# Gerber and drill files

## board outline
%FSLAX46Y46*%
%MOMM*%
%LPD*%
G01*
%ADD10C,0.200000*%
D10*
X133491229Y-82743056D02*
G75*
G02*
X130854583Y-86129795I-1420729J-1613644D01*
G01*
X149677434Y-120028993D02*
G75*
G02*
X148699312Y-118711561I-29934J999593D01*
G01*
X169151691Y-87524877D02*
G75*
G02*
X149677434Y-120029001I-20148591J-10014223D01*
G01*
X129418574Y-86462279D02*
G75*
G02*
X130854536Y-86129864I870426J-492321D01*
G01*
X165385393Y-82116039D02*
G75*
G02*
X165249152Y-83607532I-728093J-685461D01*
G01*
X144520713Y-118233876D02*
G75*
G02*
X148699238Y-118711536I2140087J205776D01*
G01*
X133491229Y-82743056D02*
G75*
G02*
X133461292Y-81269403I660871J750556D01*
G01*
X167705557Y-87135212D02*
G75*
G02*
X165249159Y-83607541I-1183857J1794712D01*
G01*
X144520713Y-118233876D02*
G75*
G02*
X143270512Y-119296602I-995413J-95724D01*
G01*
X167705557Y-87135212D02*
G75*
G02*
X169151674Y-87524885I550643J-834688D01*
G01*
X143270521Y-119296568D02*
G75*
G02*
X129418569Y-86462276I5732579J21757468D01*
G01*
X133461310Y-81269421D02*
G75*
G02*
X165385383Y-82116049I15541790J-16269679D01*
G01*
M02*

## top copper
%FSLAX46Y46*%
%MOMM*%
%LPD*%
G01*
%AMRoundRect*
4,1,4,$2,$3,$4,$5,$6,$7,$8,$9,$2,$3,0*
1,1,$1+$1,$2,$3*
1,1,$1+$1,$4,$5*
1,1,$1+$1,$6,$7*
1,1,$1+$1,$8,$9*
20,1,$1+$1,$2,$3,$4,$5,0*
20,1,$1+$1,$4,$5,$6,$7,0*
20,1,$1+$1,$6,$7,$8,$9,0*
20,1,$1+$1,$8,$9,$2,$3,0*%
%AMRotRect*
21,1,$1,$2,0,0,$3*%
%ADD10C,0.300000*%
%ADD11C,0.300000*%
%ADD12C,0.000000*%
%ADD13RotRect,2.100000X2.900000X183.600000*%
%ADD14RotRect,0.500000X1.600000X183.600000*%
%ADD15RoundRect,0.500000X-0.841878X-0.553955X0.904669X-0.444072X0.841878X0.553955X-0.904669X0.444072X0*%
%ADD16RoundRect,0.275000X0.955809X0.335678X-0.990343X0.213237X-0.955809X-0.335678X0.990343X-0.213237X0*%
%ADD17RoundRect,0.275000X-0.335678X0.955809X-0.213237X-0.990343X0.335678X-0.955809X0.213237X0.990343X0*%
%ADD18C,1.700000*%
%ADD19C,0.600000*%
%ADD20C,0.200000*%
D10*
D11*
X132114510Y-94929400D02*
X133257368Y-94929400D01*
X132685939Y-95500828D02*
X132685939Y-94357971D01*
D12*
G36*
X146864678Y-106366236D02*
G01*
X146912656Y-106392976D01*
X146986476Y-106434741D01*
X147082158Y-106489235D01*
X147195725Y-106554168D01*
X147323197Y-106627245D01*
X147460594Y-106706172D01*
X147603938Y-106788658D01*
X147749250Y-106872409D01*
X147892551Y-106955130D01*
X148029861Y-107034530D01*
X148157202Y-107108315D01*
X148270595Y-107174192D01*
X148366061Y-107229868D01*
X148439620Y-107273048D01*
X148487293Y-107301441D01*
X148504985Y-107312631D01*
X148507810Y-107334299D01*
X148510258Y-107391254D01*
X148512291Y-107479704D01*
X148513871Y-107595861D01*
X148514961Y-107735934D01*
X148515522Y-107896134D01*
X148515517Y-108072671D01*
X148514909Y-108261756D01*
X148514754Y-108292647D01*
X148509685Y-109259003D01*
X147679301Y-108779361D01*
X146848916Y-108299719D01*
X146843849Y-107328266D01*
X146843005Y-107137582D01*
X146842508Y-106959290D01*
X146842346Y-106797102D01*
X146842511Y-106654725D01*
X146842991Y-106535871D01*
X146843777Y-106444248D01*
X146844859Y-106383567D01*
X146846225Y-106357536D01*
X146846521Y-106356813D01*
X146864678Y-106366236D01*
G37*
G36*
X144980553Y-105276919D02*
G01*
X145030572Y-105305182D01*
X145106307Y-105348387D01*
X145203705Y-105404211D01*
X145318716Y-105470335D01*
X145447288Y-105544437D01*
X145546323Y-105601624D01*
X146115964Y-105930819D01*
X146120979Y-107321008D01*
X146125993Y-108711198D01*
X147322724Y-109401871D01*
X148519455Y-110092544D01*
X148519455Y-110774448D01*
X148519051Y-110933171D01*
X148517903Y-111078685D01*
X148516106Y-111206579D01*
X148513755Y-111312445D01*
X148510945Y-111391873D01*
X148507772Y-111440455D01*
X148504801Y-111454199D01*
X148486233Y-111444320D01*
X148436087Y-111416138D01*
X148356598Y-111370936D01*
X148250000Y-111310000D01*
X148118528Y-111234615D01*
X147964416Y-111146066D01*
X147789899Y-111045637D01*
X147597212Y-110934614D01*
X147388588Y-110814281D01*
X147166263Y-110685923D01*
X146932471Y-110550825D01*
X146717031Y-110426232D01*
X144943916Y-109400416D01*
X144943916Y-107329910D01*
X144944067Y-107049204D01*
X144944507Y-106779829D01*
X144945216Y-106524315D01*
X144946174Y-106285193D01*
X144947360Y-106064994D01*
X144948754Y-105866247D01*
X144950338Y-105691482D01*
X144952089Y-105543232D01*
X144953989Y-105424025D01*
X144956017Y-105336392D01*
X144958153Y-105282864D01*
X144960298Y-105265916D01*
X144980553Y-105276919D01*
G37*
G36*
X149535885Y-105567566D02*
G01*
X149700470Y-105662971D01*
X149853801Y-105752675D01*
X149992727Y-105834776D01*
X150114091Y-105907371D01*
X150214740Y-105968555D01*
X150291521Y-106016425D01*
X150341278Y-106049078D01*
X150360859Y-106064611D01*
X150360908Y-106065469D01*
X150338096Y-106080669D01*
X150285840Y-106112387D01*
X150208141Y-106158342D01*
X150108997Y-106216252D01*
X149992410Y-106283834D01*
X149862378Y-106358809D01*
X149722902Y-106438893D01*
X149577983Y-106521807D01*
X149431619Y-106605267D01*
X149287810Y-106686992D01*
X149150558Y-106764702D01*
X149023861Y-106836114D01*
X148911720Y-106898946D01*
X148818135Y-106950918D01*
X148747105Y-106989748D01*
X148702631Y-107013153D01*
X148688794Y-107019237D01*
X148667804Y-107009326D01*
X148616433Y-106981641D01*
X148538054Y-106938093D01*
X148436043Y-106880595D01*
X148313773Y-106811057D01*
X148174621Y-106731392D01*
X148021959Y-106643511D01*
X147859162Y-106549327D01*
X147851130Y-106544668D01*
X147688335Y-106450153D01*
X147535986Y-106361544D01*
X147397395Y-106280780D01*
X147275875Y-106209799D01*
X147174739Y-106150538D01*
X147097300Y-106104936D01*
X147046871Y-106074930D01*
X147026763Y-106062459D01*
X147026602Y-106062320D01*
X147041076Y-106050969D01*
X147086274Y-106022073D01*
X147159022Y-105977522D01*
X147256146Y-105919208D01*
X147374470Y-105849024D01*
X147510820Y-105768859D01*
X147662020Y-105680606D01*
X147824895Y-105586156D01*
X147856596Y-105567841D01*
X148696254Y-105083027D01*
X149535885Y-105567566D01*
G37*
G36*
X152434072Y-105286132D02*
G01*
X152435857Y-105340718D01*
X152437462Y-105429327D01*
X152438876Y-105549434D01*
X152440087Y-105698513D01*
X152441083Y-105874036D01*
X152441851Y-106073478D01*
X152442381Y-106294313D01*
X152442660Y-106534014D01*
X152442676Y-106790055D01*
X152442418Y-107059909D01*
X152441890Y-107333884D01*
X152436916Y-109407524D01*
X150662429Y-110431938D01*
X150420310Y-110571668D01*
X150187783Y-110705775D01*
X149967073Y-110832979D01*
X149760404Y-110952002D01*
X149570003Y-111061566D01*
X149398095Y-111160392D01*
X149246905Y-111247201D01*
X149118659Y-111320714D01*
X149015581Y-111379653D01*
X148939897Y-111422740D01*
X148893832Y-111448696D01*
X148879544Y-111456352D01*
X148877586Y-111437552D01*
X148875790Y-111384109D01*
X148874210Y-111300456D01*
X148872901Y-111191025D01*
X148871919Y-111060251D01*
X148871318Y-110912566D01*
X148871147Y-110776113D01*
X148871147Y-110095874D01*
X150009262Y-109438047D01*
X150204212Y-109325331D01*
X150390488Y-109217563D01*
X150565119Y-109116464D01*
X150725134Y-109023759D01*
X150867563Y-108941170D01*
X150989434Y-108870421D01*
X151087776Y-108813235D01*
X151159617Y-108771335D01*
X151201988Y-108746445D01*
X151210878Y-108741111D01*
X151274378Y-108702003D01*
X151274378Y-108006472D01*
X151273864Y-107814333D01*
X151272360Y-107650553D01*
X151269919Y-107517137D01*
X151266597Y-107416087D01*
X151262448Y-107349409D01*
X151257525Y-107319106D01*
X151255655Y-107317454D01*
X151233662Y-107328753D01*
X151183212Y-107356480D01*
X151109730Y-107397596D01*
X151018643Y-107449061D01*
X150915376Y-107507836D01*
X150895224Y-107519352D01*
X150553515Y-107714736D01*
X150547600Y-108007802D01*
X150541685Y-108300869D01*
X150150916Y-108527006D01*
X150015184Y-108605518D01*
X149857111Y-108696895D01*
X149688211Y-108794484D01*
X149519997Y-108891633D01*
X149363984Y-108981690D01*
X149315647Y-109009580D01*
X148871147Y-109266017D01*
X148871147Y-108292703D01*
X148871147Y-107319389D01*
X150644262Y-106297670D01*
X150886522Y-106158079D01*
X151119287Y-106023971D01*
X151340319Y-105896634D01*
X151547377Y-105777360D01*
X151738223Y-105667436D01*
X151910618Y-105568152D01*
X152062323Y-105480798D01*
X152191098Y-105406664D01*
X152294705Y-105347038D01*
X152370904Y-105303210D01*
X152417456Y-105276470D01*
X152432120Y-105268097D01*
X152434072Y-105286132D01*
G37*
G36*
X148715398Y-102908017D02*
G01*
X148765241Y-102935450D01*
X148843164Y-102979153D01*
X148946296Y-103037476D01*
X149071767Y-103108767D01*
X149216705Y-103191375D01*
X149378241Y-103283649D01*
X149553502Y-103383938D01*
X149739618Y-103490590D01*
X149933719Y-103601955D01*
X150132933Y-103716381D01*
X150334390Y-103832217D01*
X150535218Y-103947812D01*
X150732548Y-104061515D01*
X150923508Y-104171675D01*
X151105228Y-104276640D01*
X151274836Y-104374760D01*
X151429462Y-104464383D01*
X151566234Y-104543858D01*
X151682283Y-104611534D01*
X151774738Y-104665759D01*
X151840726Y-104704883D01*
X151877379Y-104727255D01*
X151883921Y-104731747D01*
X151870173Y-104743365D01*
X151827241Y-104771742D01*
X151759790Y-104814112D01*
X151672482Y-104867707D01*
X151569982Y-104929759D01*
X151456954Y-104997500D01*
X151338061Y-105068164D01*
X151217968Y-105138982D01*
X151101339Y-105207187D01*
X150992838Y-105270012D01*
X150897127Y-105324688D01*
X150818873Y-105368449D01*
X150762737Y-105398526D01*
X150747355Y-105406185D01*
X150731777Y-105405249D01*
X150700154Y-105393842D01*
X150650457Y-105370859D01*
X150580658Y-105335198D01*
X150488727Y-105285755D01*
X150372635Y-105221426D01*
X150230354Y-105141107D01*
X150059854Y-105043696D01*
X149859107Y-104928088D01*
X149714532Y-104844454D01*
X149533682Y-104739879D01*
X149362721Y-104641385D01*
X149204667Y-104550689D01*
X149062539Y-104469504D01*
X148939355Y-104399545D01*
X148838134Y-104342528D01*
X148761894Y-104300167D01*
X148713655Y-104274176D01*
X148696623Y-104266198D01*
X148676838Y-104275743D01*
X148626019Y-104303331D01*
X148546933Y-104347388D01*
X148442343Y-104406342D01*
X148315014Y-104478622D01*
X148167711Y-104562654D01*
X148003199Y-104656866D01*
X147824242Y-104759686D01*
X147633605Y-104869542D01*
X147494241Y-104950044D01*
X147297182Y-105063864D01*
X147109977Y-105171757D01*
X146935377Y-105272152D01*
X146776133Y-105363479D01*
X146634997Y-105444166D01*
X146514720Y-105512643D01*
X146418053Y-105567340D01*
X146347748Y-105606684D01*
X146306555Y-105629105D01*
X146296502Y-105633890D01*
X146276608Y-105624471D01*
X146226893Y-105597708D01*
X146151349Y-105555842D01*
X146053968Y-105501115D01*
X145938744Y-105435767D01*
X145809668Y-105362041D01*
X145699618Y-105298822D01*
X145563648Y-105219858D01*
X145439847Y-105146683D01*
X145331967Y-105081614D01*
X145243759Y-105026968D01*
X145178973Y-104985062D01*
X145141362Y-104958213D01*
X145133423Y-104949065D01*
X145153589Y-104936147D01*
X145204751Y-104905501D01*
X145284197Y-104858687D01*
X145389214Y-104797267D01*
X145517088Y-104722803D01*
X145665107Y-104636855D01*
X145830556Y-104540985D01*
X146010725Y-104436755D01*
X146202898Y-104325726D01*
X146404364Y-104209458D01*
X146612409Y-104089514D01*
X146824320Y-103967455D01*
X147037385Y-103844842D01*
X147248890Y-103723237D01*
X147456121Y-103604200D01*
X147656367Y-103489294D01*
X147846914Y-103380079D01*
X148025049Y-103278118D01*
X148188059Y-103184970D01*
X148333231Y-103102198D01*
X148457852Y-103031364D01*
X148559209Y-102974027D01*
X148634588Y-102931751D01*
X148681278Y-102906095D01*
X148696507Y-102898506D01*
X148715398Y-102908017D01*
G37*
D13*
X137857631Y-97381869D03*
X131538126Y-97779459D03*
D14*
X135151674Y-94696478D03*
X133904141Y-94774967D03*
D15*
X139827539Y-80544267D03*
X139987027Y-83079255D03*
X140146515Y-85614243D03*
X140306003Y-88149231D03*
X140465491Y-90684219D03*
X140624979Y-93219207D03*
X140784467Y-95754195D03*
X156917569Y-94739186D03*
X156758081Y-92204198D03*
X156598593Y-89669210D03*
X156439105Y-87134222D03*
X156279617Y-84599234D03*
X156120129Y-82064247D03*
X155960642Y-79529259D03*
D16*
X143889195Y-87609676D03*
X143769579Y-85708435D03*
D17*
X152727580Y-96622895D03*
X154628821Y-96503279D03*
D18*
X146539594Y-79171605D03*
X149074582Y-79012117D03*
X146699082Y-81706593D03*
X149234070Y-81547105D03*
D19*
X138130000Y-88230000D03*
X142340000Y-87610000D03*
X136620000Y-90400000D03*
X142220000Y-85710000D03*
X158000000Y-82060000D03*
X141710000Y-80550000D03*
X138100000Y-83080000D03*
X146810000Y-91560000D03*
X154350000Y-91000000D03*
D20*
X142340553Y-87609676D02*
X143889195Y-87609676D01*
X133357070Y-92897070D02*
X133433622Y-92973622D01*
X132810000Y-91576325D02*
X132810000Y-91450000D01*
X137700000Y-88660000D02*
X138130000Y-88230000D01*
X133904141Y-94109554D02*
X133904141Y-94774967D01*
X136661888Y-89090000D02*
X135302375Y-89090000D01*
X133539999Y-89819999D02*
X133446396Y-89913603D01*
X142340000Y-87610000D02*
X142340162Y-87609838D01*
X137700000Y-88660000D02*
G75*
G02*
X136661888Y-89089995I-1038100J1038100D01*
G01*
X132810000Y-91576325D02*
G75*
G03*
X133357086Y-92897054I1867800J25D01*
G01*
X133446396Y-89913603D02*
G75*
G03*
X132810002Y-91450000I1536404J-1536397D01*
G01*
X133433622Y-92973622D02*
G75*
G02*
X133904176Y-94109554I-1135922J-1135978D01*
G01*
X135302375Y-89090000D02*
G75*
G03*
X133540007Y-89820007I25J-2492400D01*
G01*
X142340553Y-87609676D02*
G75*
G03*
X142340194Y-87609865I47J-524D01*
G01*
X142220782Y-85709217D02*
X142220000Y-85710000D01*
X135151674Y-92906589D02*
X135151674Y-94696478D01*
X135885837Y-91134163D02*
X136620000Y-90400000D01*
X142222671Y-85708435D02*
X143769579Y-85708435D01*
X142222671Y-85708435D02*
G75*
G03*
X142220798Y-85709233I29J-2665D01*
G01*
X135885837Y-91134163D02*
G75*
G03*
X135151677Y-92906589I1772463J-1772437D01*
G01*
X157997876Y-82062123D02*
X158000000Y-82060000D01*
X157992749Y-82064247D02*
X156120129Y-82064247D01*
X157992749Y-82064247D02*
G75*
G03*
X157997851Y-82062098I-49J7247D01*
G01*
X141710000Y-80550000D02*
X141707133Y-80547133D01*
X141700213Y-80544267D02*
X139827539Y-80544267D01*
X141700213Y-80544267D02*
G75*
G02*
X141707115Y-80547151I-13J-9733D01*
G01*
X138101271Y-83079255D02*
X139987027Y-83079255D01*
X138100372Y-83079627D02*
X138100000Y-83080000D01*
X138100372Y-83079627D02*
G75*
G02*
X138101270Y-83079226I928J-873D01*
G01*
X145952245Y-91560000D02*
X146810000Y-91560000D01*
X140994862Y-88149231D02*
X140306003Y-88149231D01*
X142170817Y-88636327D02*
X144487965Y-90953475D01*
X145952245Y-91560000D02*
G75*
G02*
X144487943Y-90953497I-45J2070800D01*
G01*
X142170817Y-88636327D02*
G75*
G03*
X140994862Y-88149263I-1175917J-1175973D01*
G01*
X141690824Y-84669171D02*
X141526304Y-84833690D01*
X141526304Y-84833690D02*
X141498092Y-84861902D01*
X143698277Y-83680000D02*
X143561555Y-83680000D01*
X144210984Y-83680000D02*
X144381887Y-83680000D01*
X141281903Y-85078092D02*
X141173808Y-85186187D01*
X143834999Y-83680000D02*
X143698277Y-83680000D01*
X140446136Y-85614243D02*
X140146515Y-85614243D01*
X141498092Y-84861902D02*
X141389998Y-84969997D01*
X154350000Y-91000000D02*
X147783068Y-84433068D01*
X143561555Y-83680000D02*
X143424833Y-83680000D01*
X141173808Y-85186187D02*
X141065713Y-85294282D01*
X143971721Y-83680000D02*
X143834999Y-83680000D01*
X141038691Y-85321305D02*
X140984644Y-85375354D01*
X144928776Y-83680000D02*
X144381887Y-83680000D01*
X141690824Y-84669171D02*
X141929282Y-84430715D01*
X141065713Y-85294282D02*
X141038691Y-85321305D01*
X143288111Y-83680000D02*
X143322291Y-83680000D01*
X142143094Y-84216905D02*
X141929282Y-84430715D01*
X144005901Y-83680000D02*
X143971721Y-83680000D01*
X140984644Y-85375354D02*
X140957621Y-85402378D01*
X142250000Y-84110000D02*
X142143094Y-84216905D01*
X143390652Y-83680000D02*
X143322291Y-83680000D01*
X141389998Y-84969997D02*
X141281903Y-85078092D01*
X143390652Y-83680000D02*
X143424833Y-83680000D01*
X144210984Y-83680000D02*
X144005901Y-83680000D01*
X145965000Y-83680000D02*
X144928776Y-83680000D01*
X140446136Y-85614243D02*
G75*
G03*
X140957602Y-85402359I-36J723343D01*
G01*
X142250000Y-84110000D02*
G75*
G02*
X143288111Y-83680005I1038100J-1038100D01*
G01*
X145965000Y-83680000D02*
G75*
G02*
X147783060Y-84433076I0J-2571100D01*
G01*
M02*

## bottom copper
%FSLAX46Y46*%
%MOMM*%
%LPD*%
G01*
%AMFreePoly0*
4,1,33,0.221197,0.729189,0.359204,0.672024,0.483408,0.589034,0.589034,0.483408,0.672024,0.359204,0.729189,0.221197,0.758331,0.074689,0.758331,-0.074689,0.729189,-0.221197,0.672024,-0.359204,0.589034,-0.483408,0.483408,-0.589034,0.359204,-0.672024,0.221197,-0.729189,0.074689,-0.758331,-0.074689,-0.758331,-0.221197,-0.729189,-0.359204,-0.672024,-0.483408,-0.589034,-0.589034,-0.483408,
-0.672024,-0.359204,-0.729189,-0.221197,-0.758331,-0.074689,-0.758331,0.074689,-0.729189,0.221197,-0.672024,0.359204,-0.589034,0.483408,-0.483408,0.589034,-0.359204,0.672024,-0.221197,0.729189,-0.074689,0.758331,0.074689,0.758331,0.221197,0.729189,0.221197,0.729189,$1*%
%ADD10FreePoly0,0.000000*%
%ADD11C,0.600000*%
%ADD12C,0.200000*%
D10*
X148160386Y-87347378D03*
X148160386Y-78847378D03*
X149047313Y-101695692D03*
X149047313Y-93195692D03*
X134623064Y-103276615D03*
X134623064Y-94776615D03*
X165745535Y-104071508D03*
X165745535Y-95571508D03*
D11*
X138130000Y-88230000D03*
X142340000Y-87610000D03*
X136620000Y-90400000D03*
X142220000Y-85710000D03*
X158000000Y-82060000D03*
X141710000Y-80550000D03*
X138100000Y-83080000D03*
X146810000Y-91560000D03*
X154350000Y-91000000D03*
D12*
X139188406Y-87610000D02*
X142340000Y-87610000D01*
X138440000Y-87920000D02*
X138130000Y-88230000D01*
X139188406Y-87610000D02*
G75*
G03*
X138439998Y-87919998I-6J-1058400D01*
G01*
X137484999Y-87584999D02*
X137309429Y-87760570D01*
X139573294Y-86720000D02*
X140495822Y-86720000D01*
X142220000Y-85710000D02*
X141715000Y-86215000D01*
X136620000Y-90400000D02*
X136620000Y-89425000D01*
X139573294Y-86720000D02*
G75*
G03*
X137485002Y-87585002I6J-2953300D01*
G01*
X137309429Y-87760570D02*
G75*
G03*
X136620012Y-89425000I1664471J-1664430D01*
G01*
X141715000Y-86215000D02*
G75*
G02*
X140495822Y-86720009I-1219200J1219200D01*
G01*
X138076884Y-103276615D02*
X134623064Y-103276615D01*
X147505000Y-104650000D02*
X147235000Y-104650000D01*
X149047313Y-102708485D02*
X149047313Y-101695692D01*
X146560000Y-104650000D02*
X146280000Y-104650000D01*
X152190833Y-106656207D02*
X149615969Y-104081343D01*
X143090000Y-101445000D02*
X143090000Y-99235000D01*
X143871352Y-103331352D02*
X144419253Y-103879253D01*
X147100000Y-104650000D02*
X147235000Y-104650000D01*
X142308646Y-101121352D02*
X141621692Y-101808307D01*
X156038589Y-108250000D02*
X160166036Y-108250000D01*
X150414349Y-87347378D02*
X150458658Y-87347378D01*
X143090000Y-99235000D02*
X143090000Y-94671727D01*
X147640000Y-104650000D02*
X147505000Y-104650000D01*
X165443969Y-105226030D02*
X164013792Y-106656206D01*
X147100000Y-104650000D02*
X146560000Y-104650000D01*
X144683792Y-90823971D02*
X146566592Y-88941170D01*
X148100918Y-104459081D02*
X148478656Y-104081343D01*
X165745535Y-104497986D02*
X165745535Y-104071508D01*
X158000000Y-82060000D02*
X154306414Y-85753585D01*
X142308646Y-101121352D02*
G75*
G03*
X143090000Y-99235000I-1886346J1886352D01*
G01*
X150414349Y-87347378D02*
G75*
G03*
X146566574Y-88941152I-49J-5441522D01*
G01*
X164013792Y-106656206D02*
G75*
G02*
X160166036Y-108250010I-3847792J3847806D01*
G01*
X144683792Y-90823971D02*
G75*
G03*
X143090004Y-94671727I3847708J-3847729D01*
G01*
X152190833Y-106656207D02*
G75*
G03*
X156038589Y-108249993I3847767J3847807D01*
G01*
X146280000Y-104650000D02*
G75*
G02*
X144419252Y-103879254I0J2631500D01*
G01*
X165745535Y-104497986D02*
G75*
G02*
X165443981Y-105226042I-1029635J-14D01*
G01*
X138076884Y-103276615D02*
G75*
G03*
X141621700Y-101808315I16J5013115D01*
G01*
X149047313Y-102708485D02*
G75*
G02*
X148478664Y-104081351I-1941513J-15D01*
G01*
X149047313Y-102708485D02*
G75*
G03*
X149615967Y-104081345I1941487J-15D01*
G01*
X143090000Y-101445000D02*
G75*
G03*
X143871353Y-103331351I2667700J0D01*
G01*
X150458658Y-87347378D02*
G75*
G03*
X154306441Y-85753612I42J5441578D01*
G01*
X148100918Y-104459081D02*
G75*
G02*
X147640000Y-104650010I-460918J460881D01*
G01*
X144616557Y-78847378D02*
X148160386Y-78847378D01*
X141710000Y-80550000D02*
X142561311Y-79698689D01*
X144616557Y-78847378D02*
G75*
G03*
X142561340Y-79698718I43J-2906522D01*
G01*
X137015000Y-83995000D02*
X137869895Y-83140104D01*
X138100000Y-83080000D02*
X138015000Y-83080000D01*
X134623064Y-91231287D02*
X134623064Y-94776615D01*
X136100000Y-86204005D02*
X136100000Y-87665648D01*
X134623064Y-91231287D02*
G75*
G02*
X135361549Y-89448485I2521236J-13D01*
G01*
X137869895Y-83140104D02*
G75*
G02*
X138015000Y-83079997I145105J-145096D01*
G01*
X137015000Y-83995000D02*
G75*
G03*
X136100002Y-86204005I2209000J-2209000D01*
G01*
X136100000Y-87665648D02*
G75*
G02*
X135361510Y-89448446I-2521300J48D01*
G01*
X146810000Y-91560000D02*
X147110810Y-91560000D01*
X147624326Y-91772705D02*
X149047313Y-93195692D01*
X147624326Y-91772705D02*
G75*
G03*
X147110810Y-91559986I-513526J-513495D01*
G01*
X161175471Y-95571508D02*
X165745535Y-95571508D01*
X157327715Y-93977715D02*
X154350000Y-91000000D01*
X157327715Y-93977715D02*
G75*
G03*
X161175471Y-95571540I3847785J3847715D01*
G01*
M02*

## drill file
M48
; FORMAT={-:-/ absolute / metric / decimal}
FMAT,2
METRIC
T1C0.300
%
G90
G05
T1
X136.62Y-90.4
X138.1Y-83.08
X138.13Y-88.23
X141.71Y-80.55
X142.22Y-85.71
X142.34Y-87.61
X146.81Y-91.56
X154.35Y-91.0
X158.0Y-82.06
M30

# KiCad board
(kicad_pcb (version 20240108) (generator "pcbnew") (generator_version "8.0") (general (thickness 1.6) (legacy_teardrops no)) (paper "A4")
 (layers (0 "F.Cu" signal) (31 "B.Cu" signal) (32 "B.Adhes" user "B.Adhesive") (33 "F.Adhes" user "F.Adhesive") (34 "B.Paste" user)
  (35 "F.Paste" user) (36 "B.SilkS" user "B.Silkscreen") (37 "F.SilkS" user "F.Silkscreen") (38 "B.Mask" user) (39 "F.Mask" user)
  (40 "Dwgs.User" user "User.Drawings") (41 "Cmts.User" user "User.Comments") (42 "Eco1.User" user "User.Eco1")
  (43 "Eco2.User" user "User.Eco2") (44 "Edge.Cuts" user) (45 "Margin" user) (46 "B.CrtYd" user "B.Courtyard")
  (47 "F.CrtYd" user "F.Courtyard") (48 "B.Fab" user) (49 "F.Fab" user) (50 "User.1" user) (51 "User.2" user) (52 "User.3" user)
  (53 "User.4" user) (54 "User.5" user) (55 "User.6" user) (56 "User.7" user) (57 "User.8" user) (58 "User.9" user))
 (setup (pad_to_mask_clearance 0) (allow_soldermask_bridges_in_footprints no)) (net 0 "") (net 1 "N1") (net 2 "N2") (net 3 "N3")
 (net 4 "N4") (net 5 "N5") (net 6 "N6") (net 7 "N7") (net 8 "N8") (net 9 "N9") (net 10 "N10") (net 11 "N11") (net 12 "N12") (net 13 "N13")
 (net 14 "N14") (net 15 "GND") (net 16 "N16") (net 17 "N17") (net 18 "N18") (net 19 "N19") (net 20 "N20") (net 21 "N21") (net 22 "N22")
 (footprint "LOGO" (layer "F.Cu") (at 148.7 107.18)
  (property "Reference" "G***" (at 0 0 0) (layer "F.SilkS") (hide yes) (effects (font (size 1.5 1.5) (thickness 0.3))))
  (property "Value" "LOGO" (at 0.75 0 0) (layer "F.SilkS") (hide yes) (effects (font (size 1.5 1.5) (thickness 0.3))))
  (fp_poly
   (pts (xy -1.835322 -0.813764) (xy -1.787344 -0.787024) (xy -1.713524 -0.745259) (xy -1.617842 -0.690765) (xy -1.504275 -0.625832)
    (xy -1.376803 -0.552755) (xy -1.239406 -0.473828) (xy -1.096062 -0.391342) (xy -0.95075 -0.307591) (xy -0.807449 -0.22487)
    (xy -0.670139 -0.14547) (xy -0.542798 -0.071685) (xy -0.429405 -0.005808) (xy -0.333939 0.049868) (xy -0.26038 0.093048)
    (xy -0.212707 0.121441) (xy -0.195015 0.132631) (xy -0.19219 0.154299) (xy -0.189742 0.211254) (xy -0.187709 0.299704)
    (xy -0.186129 0.415861) (xy -0.185039 0.555934) (xy -0.184478 0.716134) (xy -0.184483 0.892671) (xy -0.185091 1.081756)
    (xy -0.185246 1.112647) (xy -0.190315 2.079003) (xy -1.020699 1.599361) (xy -1.851084 1.119719) (xy -1.856151 0.148266)
    (xy -1.856995 -0.042418) (xy -1.857492 -0.22071) (xy -1.857654 -0.382898) (xy -1.857489 -0.525275) (xy -1.857009 -0.644129)
    (xy -1.856223 -0.735752) (xy -1.855141 -0.796433) (xy -1.853775 -0.822464) (xy -1.853479 -0.823187))
   (stroke (width 0) (type solid)) (fill solid) (layer "F.Cu"))
  (fp_poly
   (pts (xy -3.719447 -1.903081) (xy -3.669428 -1.874818) (xy -3.593693 -1.831613) (xy -3.496295 -1.775789) (xy -3.381284 -1.709665)
    (xy -3.252712 -1.635563) (xy -3.153677 -1.578376) (xy -2.584036 -1.249181) (xy -2.579021 0.141008) (xy -2.574007 1.531198)
    (xy -1.377276 2.221871) (xy -0.180545 2.912544) (xy -0.180545 3.594448) (xy -0.180949 3.753171) (xy -0.182097 3.898685)
    (xy -0.183894 4.026579) (xy -0.186245 4.132445) (xy -0.189055 4.211873) (xy -0.192228 4.260455) (xy -0.195199 4.274199)
    (xy -0.213767 4.26432) (xy -0.263913 4.236138) (xy -0.343402 4.190936) (xy -0.45 4.13) (xy -0.581472 4.054615) (xy -0.735584 3.966066)
    (xy -0.910101 3.865637) (xy -1.102788 3.754614) (xy -1.311412 3.634281) (xy -1.533737 3.505923) (xy -1.767529 3.370825)
    (xy -1.982969 3.246232) (xy -3.756084 2.220416) (xy -3.756084 0.14991) (xy -3.755933 -0.130796) (xy -3.755493 -0.400171)
    (xy -3.754784 -0.655685) (xy -3.753826 -0.894807) (xy -3.75264 -1.115006) (xy -3.751246 -1.313753) (xy -3.749662 -1.488518)
    (xy -3.747911 -1.636768) (xy -3.746011 -1.755975) (xy -3.743983 -1.843608) (xy -3.741847 -1.897136) (xy -3.739702 -1.914084))
   (stroke (width 0) (type solid)) (fill solid) (layer "F.Cu"))
  (fp_poly
   (pts (xy 0.835885 -1.612434) (xy 1.00047 -1.517029) (xy 1.153801 -1.427325) (xy 1.292727 -1.345224) (xy 1.414091 -1.272629)
    (xy 1.51474 -1.211445) (xy 1.591521 -1.163575) (xy 1.641278 -1.130922) (xy 1.660859 -1.115389) (xy 1.660908 -1.114531)
    (xy 1.638096 -1.099331) (xy 1.58584 -1.067613) (xy 1.508141 -1.021658) (xy 1.408997 -0.963748) (xy 1.29241 -0.896166)
    (xy 1.162378 -0.821191) (xy 1.022902 -0.741107) (xy 0.877983 -0.658193) (xy 0.731619 -0.574733) (xy 0.58781 -0.493008)
    (xy 0.450558 -0.415298) (xy 0.323861 -0.343886) (xy 0.21172 -0.281054) (xy 0.118135 -0.229082) (xy 0.047105 -0.190252)
    (xy 0.002631 -0.166847) (xy -0.011206 -0.160763) (xy -0.032196 -0.170674) (xy -0.083567 -0.198359) (xy -0.161946 -0.241907)
    (xy -0.263957 -0.299405) (xy -0.386227 -0.368943) (xy -0.525379 -0.448608) (xy -0.678041 -0.536489) (xy -0.840838 -0.630673)
    (xy -0.84887 -0.635332) (xy -1.011665 -0.729847) (xy -1.164014 -0.818456) (xy -1.302605 -0.89922) (xy -1.424125 -0.970201)
    (xy -1.525261 -1.029462) (xy -1.6027 -1.075064) (xy -1.653129 -1.10507) (xy -1.673237 -1.117541) (xy -1.673398 -1.11768)
    (xy -1.658924 -1.129031) (xy -1.613726 -1.157927) (xy -1.540978 -1.202478) (xy -1.443854 -1.260792) (xy -1.32553 -1.330976)
    (xy -1.18918 -1.411141) (xy -1.03798 -1.499394) (xy -0.875105 -1.593844) (xy -0.843404 -1.612159) (xy -0.003746 -2.096973))
   (stroke (width 0) (type solid)) (fill solid) (layer "F.Cu"))
  (fp_poly
   (pts (xy 3.734072 -1.893868) (xy 3.735857 -1.839282) (xy 3.737462 -1.750673) (xy 3.738876 -1.630566) (xy 3.740087 -1.481487)
    (xy 3.741083 -1.305964) (xy 3.741851 -1.106522) (xy 3.742381 -0.885687) (xy 3.74266 -0.645986) (xy 3.742676 -0.389945)
    (xy 3.742418 -0.120091) (xy 3.74189 0.153884) (xy 3.736916 2.227524) (xy 1.962429 3.251938) (xy 1.72031 3.391668) (xy 1.487783 3.525775)
    (xy 1.267073 3.652979) (xy 1.060404 3.772002) (xy 0.870003 3.881566) (xy 0.698095 3.980392) (xy 0.546905 4.067201)
    (xy 0.418659 4.140714) (xy 0.315581 4.199653) (xy 0.239897 4.24274) (xy 0.193832 4.268696) (xy 0.179544 4.276352) (xy 0.177586 4.257552)
    (xy 0.17579 4.204109) (xy 0.17421 4.120456) (xy 0.172901 4.011025) (xy 0.171919 3.880251) (xy 0.171318 3.732566) (xy 0.171147 3.596113)
    (xy 0.171147 2.915874) (xy 1.309262 2.258047) (xy 1.504212 2.145331) (xy 1.690488 2.037563) (xy 1.865119 1.936464)
    (xy 2.025134 1.843759) (xy 2.167563 1.76117) (xy 2.289434 1.690421) (xy 2.387776 1.633235) (xy 2.459617 1.591335) (xy 2.501988 1.566445)
    (xy 2.510878 1.561111) (xy 2.574378 1.522003) (xy 2.574378 0.826472) (xy 2.573864 0.634333) (xy 2.57236 0.470553) (xy 2.569919 0.337137)
    (xy 2.566597 0.236087) (xy 2.562448 0.169409) (xy 2.557525 0.139106) (xy 2.555655 0.137454) (xy 2.533662 0.148753) (xy 2.483212 0.17648)
    (xy 2.40973 0.217596) (xy 2.318643 0.269061) (xy 2.215376 0.327836) (xy 2.195224 0.339352) (xy 1.853515 0.534736) (xy 1.8476 0.827802)
    (xy 1.841685 1.120869) (xy 1.450916 1.347006) (xy 1.315184 1.425518) (xy 1.157111 1.516895) (xy 0.988211 1.614484)
    (xy 0.819997 1.711633) (xy 0.663984 1.80169) (xy 0.615647 1.82958) (xy 0.171147 2.086017) (xy 0.171147 1.112703) (xy 0.171147 0.139389)
    (xy 1.944262 -0.88233) (xy 2.186522 -1.021921) (xy 2.419287 -1.156029) (xy 2.640319 -1.283366) (xy 2.847377 -1.40264)
    (xy 3.038223 -1.512564) (xy 3.210618 -1.611848) (xy 3.362323 -1.699202) (xy 3.491098 -1.773336) (xy 3.594705 -1.832962)
    (xy 3.670904 -1.87679) (xy 3.717456 -1.90353) (xy 3.73212 -1.911903))
   (stroke (width 0) (type solid)) (fill solid) (layer "F.Cu"))
  (fp_poly
   (pts (xy 0.015398 -4.271983) (xy 0.065241 -4.24455) (xy 0.143164 -4.200847) (xy 0.246296 -4.142524) (xy 0.371767 -4.071233)
    (xy 0.516705 -3.988625) (xy 0.678241 -3.896351) (xy 0.853502 -3.796062) (xy 1.039618 -3.68941) (xy 1.233719 -3.578045)
    (xy 1.432933 -3.463619) (xy 1.63439 -3.347783) (xy 1.835218 -3.232188) (xy 2.032548 -3.118485) (xy 2.223508 -3.008325)
    (xy 2.405228 -2.90336) (xy 2.574836 -2.80524) (xy 2.729462 -2.715617) (xy 2.866234 -2.636142) (xy 2.982283 -2.568466)
    (xy 3.074738 -2.514241) (xy 3.140726 -2.475117) (xy 3.177379 -2.452745) (xy 3.183921 -2.448253) (xy 3.170173 -2.436635)
    (xy 3.127241 -2.408258) (xy 3.05979 -2.365888) (xy 2.972482 -2.312293) (xy 2.869982 -2.250241) (xy 2.756954 -2.1825)
    (xy 2.638061 -2.111836) (xy 2.517968 -2.041018) (xy 2.401339 -1.972813) (xy 2.292838 -1.909988) (xy 2.197127 -1.855312)
    (xy 2.118873 -1.811551) (xy 2.062737 -1.781474) (xy 2.047355 -1.773815) (xy 2.031777 -1.774751) (xy 2.000154 -1.786158)
    (xy 1.950457 -1.809141) (xy 1.880658 -1.844802) (xy 1.788727 -1.894245) (xy 1.672635 -1.958574) (xy 1.530354 -2.038893)
    (xy 1.359854 -2.136304) (xy 1.159107 -2.251912) (xy 1.014532 -2.335546) (xy 0.833682 -2.440121) (xy 0.662721 -2.538615)
    (xy 0.504667 -2.629311) (xy 0.362539 -2.710496) (xy 0.239355 -2.780455) (xy 0.138134 -2.837472) (xy 0.061894 -2.879833)
    (xy 0.013655 -2.905824) (xy -0.003377 -2.913802) (xy -0.023162 -2.904257) (xy -0.073981 -2.876669) (xy -0.153067 -2.832612)
    (xy -0.257657 -2.773658) (xy -0.384986 -2.701378) (xy -0.532289 -2.617346) (xy -0.696801 -2.523134) (xy -0.875758 -2.420314)
    (xy -1.066395 -2.310458) (xy -1.205759 -2.229956) (xy -1.402818 -2.116136) (xy -1.590023 -2.008243) (xy -1.764623 -1.907848)
    (xy -1.923867 -1.816521) (xy -2.065003 -1.735834) (xy -2.18528 -1.667357) (xy -2.281947 -1.61266) (xy -2.352252 -1.573316)
    (xy -2.393445 -1.550895) (xy -2.403498 -1.54611) (xy -2.423392 -1.555529) (xy -2.473107 -1.582292) (xy -2.548651 -1.624158)
    (xy -2.646032 -1.678885) (xy -2.761256 -1.744233) (xy -2.890332 -1.817959) (xy -3.000382 -1.881178) (xy -3.136352 -1.960142)
    (xy -3.260153 -2.033317) (xy -3.368033 -2.098386) (xy -3.456241 -2.153032) (xy -3.521027 -2.194938) (xy -3.558638 -2.221787)
    (xy -3.566577 -2.230935) (xy -3.546411 -2.243853) (xy -3.495249 -2.274499) (xy -3.415803 -2.321313) (xy -3.310786 -2.382733)
    (xy -3.182912 -2.457197) (xy -3.034893 -2.543145) (xy -2.869444 -2.639015) (xy -2.689275 -2.743245) (xy -2.497102 -2.854274)
    (xy -2.295636 -2.970542) (xy -2.087591 -3.090486) (xy -1.87568 -3.212545) (xy -1.662615 -3.335158) (xy -1.45111 -3.456763)
    (xy -1.243879 -3.5758) (xy -1.043633 -3.690706) (xy -0.853086 -3.799921) (xy -0.674951 -3.901882) (xy -0.511941 -3.99503)
    (xy -0.366769 -4.077802) (xy -0.242148 -4.148636) (xy -0.140791 -4.205973) (xy -0.065412 -4.248249) (xy -0.018722 -4.273905)
    (xy -0.003493 -4.281494))
   (stroke (width 0) (type solid)) (fill solid) (layer "F.Cu")))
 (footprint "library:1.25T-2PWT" (layer "F.Cu") (at 134.71 97.63 -176.4)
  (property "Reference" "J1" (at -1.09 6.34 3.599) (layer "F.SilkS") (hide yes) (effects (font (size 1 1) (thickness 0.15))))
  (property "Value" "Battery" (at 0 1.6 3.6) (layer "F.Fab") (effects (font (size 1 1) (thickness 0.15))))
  (pad "" smd rect (at -3.157 0.05 183.6) (size 2.1 2.9) (layers "F.Cu" "F.Paste" "F.Mask"))
  (pad "" smd rect (at 3.175 0.05 183.6) (size 2.1 2.9) (layers "F.Cu" "F.Paste" "F.Mask"))
  (pad "1" smd rect (at -0.625 2.9 183.6) (size 0.5 1.6) (layers "F.Cu" "F.Paste" "F.Mask") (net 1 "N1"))
  (pad "2" smd rect (at 0.625 2.9 183.6) (size 0.5 1.6) (layers "F.Cu" "F.Paste" "F.Mask") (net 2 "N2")))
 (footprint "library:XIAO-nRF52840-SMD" (layer "F.Cu") (at 148.4 87.64 3.6)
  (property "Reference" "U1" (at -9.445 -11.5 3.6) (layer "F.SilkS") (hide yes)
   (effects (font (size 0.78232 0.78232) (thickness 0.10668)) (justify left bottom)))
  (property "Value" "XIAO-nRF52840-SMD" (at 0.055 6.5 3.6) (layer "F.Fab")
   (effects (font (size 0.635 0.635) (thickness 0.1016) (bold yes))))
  (pad "1" smd roundrect (at -8.11 -7.62 3.6) (size 2.75 2) (layers "F.Cu" "F.Paste" "F.Mask") (roundrect_rratio 0.25) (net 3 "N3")
   (solder_mask_margin 0.0508) (thermal_bridge_angle 45))
  (pad "2" smd roundrect (at -8.11 -5.08 3.6) (size 2.75 2) (layers "F.Cu" "F.Paste" "F.Mask") (roundrect_rratio 0.25) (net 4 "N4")
   (solder_mask_margin 0.0508) (thermal_bridge_angle 45))
  (pad "3" smd roundrect (at -8.11 -2.54 3.6) (size 2.75 2) (layers "F.Cu" "F.Paste" "F.Mask") (roundrect_rratio 0.25) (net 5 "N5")
   (solder_mask_margin 0.0508) (thermal_bridge_angle 45))
  (pad "4" smd roundrect (at -8.11 0 3.6) (size 2.75 2) (layers "F.Cu" "F.Paste" "F.Mask") (roundrect_rratio 0.25) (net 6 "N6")
   (solder_mask_margin 0.0508) (thermal_bridge_angle 45))
  (pad "5" smd roundrect (at -8.11 2.54 3.6) (size 2.75 2) (layers "F.Cu" "F.Paste" "F.Mask") (roundrect_rratio 0.25) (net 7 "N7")
   (solder_mask_margin 0.0508) (thermal_bridge_angle 45))
  (pad "6" smd roundrect (at -8.11 5.08 3.6) (size 2.75 2) (layers "F.Cu" "F.Paste" "F.Mask") (roundrect_rratio 0.25) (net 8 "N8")
   (solder_mask_margin 0.0508) (thermal_bridge_angle 45))
  (pad "7" smd roundrect (at -8.11 7.62 3.6) (size 2.75 2) (layers "F.Cu" "F.Paste" "F.Mask") (roundrect_rratio 0.25) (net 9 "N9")
   (solder_mask_margin 0.0508) (thermal_bridge_angle 45))
  (pad "8" smd roundrect (at 8.055 7.62 3.6) (size 2.75 2) (layers "F.Cu" "F.Paste" "F.Mask") (roundrect_rratio 0.25) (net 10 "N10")
   (solder_mask_margin 0.0508) (thermal_bridge_angle 45))
  (pad "9" smd roundrect (at 8.055 5.08 3.6) (size 2.75 2) (layers "F.Cu" "F.Paste" "F.Mask") (roundrect_rratio 0.25) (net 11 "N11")
   (solder_mask_margin 0.0508) (thermal_bridge_angle 45))
  (pad "10" smd roundrect (at 8.055 2.54 3.6) (size 2.75 2) (layers "F.Cu" "F.Paste" "F.Mask") (roundrect_rratio 0.25) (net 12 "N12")
   (solder_mask_margin 0.0508) (thermal_bridge_angle 45))
  (pad "11" smd roundrect (at 8.055 0 3.6) (size 2.75 2) (layers "F.Cu" "F.Paste" "F.Mask") (roundrect_rratio 0.25) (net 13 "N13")
   (solder_mask_margin 0.0508) (thermal_bridge_angle 45))
  (pad "12" smd roundrect (at 8.055 -2.54 3.6) (size 2.75 2) (layers "F.Cu" "F.Paste" "F.Mask") (roundrect_rratio 0.25) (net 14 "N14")
   (solder_mask_margin 0.0508) (thermal_bridge_angle 45))
  (pad "13" smd roundrect (at 8.055 -5.08 3.6) (size 2.75 2) (layers "F.Cu" "F.Paste" "F.Mask") (roundrect_rratio 0.25) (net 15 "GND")
   (solder_mask_margin 0.0508) (thermal_bridge_angle 45))
  (pad "14" smd roundrect (at 8.055 -7.62 3.6) (size 2.75 2) (layers "F.Cu" "F.Paste" "F.Mask") (roundrect_rratio 0.25) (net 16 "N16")
   (solder_mask_margin 0.0508) (thermal_bridge_angle 45))
  (pad "15" smd roundrect (at -4.5 -0.3135 183.6) (size 2.5 1.1) (layers "F.Cu" "F.Paste" "F.Mask") (roundrect_rratio 0.25) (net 2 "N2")
   (solder_mask_margin 0.0508) (thermal_bridge_angle 45))
  (pad "16" smd roundrect (at -4.5 -2.2185 183.6) (size 2.5 1.1) (layers "F.Cu" "F.Paste" "F.Mask") (roundrect_rratio 0.25) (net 1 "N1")
   (solder_mask_margin 0.0508) (thermal_bridge_angle 45))
  (pad "17" smd roundrect (at 3.755 9.2369 273.6) (size 2.5 1.1) (layers "F.Cu" "F.Paste" "F.Mask") (roundrect_rratio 0.25) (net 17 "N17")
   (solder_mask_margin 0.0508) (thermal_bridge_angle 45))
  (pad "18" smd roundrect (at 5.66 9.2369 273.6) (size 2.5 1.1) (layers "F.Cu" "F.Paste" "F.Mask") (roundrect_rratio 0.25) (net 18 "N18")
   (solder_mask_margin 0.0508) (thermal_bridge_angle 45))
  (pad "19" smd circle (at -1.325 -8.5685 3.6) (size 1.7 1.7) (layers "F.Cu" "F.Paste" "F.Mask") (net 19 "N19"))
  (pad "20" smd circle (at 1.215 -8.5685 3.6) (size 1.7 1.7) (layers "F.Cu" "F.Paste" "F.Mask") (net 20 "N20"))
  (pad "21" smd circle (at -1.325 -6.0285 3.6) (size 1.7 1.7) (layers "F.Cu" "F.Paste" "F.Mask") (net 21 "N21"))
  (pad "22" smd circle (at 1.215 -6.0285 3.6) (size 1.7 1.7) (layers "F.Cu" "F.Paste" "F.Mask") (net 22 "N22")))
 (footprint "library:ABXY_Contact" (layer "B.Cu") (at 148.160386 83.147378)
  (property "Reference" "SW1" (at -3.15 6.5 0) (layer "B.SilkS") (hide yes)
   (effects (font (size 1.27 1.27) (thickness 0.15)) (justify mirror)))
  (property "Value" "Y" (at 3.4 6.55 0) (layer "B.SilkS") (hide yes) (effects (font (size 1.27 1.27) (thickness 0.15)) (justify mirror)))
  (pad "1" connect custom (at 0 4.2) (size 1.524 1.524) (layers "B.Cu" "B.Mask") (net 15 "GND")
   (options (clearance outline) (anchor circle)) (primitives))
  (pad "2" connect custom (at 0 -4.3) (size 1.524 1.524) (layers "B.Cu" "B.Mask") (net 3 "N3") (options (clearance outline) (anchor circle))
   (primitives)))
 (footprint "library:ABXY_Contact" (layer "B.Cu") (at 149.047313 97.495692)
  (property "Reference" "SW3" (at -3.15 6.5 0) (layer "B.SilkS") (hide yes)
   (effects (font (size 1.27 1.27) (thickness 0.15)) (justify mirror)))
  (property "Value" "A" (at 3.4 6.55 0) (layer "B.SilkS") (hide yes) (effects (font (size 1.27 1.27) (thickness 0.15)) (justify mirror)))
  (pad "1" connect custom (at 0 4.2) (size 1.524 1.524) (layers "B.Cu" "B.Mask") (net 15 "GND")
   (options (clearance outline) (anchor circle)) (primitives))
  (pad "2" connect custom (at 0 -4.3) (size 1.524 1.524) (layers "B.Cu" "B.Mask") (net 6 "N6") (options (clearance outline) (anchor circle))
   (primitives)))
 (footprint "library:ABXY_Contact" (layer "B.Cu") (at 134.623064 99.076615)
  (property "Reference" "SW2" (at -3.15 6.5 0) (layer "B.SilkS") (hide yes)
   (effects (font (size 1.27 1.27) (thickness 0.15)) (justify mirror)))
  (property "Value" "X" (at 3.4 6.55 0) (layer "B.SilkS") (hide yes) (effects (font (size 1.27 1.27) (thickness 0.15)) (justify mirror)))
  (pad "1" connect custom (at 0 4.2) (size 1.524 1.524) (layers "B.Cu" "B.Mask") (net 15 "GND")
   (options (clearance outline) (anchor circle)) (primitives))
  (pad "2" connect custom (at 0 -4.3) (size 1.524 1.524) (layers "B.Cu" "B.Mask") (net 4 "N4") (options (clearance outline) (anchor circle))
   (primitives)))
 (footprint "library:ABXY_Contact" (layer "B.Cu") (at 165.745535 99.871508)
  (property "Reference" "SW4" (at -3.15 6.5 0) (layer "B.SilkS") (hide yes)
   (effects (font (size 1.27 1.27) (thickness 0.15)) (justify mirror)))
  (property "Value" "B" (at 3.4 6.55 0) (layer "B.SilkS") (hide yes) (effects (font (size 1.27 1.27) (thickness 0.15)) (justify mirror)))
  (pad "1" connect custom (at 0 4.2) (size 1.524 1.524) (layers "B.Cu" "B.Mask") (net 15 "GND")
   (options (clearance outline) (anchor circle)) (primitives))
  (pad "2" connect custom (at 0 -4.3) (size 1.524 1.524) (layers "B.Cu" "B.Mask") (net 5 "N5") (options (clearance outline) (anchor circle))
   (primitives)))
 (gr_arc (start 133.491229 82.743056) (mid 133.766949 85.677468) (end 130.854538 86.129861) (stroke (width 0.2) (type default))
  (layer "Edge.Cuts"))
 (gr_arc (start 149.677434 120.028993) (mid 148.844558 119.625547) (end 148.699331 118.711567) (stroke (width 0.2) (type default))
  (layer "Edge.Cuts"))
 (gr_arc (start 169.151691 87.524877) (mid 168.304087 109.102934) (end 149.677434 120.028993) (stroke (width 0.2) (type default))
  (layer "Edge.Cuts"))
 (gr_arc (start 129.418574 86.462279) (mid 130.063468 85.980346) (end 130.854538 86.129861) (stroke (width 0.2) (type default))
  (layer "Edge.Cuts"))
 (gr_arc (start 165.385393 82.116039) (mid 165.653147 82.89247) (end 165.24916 83.607543) (stroke (width 0.2) (type default))
  (layer "Edge.Cuts"))
 (gr_arc (start 144.520713 118.233876) (mid 146.905039 115.892048) (end 148.699331 118.711567) (stroke (width 0.2) (type default))
  (layer "Edge.Cuts"))
 (gr_arc (start 133.491229 82.743056) (mid 133.152263 82.012817) (end 133.46131 81.269421) (stroke (width 0.2) (type default))
  (layer "Edge.Cuts"))
 (gr_arc (start 167.705557 87.135212) (mid 164.757292 86.569104) (end 165.24916 83.607543) (stroke (width 0.2) (type default))
  (layer "Edge.Cuts"))
 (gr_arc (start 144.520713 118.233876) (mid 144.172961 119.091501) (end 143.270521 119.296568) (stroke (width 0.2) (type default))
  (layer "Edge.Cuts"))
 (gr_arc (start 167.705557 87.135212) (mid 168.516386 87.004384) (end 169.151691 87.524877) (stroke (width 0.2) (type default))
  (layer "Edge.Cuts"))
 (gr_arc (start 143.270521 119.296568) (mid 128.272412 106.284851) (end 129.418574 86.462279) (stroke (width 0.2) (type default))
  (layer "Edge.Cuts"))
 (gr_arc (start 133.46131 81.269421) (mid 149.599594 75.047008) (end 165.385393 82.116039) (stroke (width 0.2) (type default))
  (layer "Edge.Cuts"))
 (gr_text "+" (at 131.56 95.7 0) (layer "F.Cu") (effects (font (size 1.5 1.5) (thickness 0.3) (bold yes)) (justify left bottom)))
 (segment (start 142.340553 87.609676) (end 143.889195 87.609676) (width 0.2) (layer "F.Cu") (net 2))
 (segment (start 133.35707 92.89707) (end 133.433622 92.973622) (width 0.2) (layer "F.Cu") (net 2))
 (segment (start 132.81 91.576325) (end 132.81 91.45) (width 0.2) (layer "F.Cu") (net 2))
 (segment (start 137.7 88.66) (end 138.13 88.23) (width 0.2) (layer "F.Cu") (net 2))
 (segment (start 133.904141 94.109554) (end 133.904141 94.774967) (width 0.2) (layer "F.Cu") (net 2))
 (segment (start 136.661888 89.09) (end 135.302375 89.09) (width 0.2) (layer "F.Cu") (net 2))
 (segment (start 133.539999 89.819999) (end 133.446396 89.913603) (width 0.2) (layer "F.Cu") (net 2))
 (segment (start 142.34 87.61) (end 142.340162 87.609838) (width 0.2) (layer "F.Cu") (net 2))
 (via (at 138.13 88.23) (size 0.6) (drill 0.3) (layers "F.Cu" "B.Cu") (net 2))
 (via (at 142.34 87.61) (size 0.6) (drill 0.3) (layers "F.Cu" "B.Cu") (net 2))
 (arc (start 137.7 88.66) (mid 137.22371 88.978246) (end 136.661888 89.09) (width 0.2) (layer "F.Cu") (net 2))
 (arc (start 132.81 91.576325) (mid 132.952178 92.291107) (end 133.35707 92.89707) (width 0.2) (layer "F.Cu") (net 2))
 (arc (start 133.446396 89.913603) (mid 132.975393 90.618508) (end 132.81 91.45) (width 0.2) (layer "F.Cu") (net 2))
 (arc (start 133.433622 92.973622) (mid 133.781857 93.494792) (end 133.904141 94.109554) (width 0.2) (layer "F.Cu") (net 2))
 (arc (start 135.302375 89.09) (mid 134.348584 89.27972) (end 133.539999 89.819999) (width 0.2) (layer "F.Cu") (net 2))
 (arc (start 142.340553 87.609676) (mid 142.340341 87.609718) (end 142.340162 87.609838) (width 0.2) (layer "F.Cu") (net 2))
 (segment (start 139.188406 87.61) (end 142.34 87.61) (width 0.2) (layer "B.Cu") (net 2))
 (segment (start 138.44 87.92) (end 138.13 88.23) (width 0.2) (layer "B.Cu") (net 2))
 (arc (start 139.188406 87.61) (mid 138.783371 87.690566) (end 138.44 87.92) (width 0.2) (layer "B.Cu") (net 2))
 (segment (start 142.220782 85.709217) (end 142.22 85.71) (width 0.2) (layer "F.Cu") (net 1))
 (segment (start 135.151674 92.906589) (end 135.151674 94.696478) (width 0.2) (layer "F.Cu") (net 1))
 (segment (start 135.885837 91.134163) (end 136.62 90.4) (width 0.2) (layer "F.Cu") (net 1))
 (segment (start 142.222671 85.708435) (end 143.769579 85.708435) (width 0.2) (layer "F.Cu") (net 1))
 (via (at 136.62 90.4) (size 0.6) (drill 0.3) (layers "F.Cu" "B.Cu") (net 1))
 (via (at 142.22 85.71) (size 0.6) (drill 0.3) (layers "F.Cu" "B.Cu") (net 1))
 (arc (start 142.222671 85.708435) (mid 142.221648 85.708638) (end 142.220782 85.709217) (width 0.2) (layer "F.Cu") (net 1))
 (arc (start 135.885837 91.134163) (mid 135.342476 91.947359) (end 135.151674 92.906589) (width 0.2) (layer "F.Cu") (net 1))
 (segment (start 137.484999 87.584999) (end 137.309429 87.76057) (width 0.2) (layer "B.Cu") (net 1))
 (segment (start 139.573294 86.72) (end 140.495822 86.72) (width 0.2) (layer "B.Cu") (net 1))
 (segment (start 142.22 85.71) (end 141.715 86.215) (width 0.2) (layer "B.Cu") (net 1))
 (segment (start 136.62 90.4) (end 136.62 89.425) (width 0.2) (layer "B.Cu") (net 1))
 (arc (start 139.573294 86.72) (mid 138.443117 86.944805) (end 137.484999 87.584999) (width 0.2) (layer "B.Cu") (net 1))
 (arc (start 137.309429 87.76057) (mid 136.799176 88.524217) (end 136.62 89.425) (width 0.2) (layer "B.Cu") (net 1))
 (arc (start 141.715 86.215) (mid 141.155636 86.588754) (end 140.495822 86.72) (width 0.2) (layer "B.Cu") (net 1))
 (segment (start 157.997876 82.062123) (end 158 82.06) (width 0.2) (layer "F.Cu") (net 15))
 (segment (start 157.992749 82.064247) (end 156.120129 82.064247) (width 0.2) (layer "F.Cu") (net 15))
 (via (at 158 82.06) (size 0.6) (drill 0.3) (layers "F.Cu" "B.Cu") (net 15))
 (arc (start 157.992749 82.064247) (mid 157.995524 82.063694) (end 157.997876 82.062123) (width 0.2) (layer "F.Cu") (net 15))
 (segment (start 138.076884 103.276615) (end 134.623064 103.276615) (width 0.2) (layer "B.Cu") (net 15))
 (segment (start 147.505 104.65) (end 147.235 104.65) (width 0.2) (layer "B.Cu") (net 15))
 (segment (start 149.047313 102.708485) (end 149.047313 101.695692) (width 0.2) (layer "B.Cu") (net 15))
 (segment (start 146.56 104.65) (end 146.28 104.65) (width 0.2) (layer "B.Cu") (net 15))
 (segment (start 152.190833 106.656207) (end 149.615969 104.081343) (width 0.2) (layer "B.Cu") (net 15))
 (segment (start 143.09 101.445) (end 143.09 99.235) (width 0.2) (layer "B.Cu") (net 15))
 (segment (start 143.871352 103.331352) (end 144.419253 103.879253) (width 0.2) (layer "B.Cu") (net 15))
 (segment (start 147.1 104.65) (end 147.235 104.65) (width 0.2) (layer "B.Cu") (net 15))
 (segment (start 142.308646 101.121352) (end 141.621692 101.808307) (width 0.2) (layer "B.Cu") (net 15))
 (segment (start 156.038589 108.25) (end 160.166036 108.25) (width 0.2) (layer "B.Cu") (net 15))
 (segment (start 150.414349 87.347378) (end 150.458658 87.347378) (width 0.2) (layer "B.Cu") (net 15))
 (segment (start 143.09 99.235) (end 143.09 94.671727) (width 0.2) (layer "B.Cu") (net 15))
 (segment (start 147.64 104.65) (end 147.505 104.65) (width 0.2) (layer "B.Cu") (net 15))
 (segment (start 165.443969 105.22603) (end 164.013792 106.656206) (width 0.2) (layer "B.Cu") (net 15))
 (segment (start 147.1 104.65) (end 146.56 104.65) (width 0.2) (layer "B.Cu") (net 15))
 (segment (start 144.683792 90.823971) (end 146.566592 88.94117) (width 0.2) (layer "B.Cu") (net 15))
 (segment (start 148.100918 104.459081) (end 148.478656 104.081343) (width 0.2) (layer "B.Cu") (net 15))
 (segment (start 165.745535 104.497986) (end 165.745535 104.071508) (width 0.2) (layer "B.Cu") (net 15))
 (segment (start 158 82.06) (end 154.306414 85.753585) (width 0.2) (layer "B.Cu") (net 15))
 (arc (start 142.308646 101.121352) (mid 142.886932 100.255886) (end 143.09 99.235) (width 0.2) (layer "B.Cu") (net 15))
 (arc (start 150.414349 87.347378) (mid 148.331958 87.761591) (end 146.566592 88.94117) (width 0.2) (layer "B.Cu") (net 15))
 (arc (start 164.013792 106.656206) (mid 162.248426 107.835786) (end 160.166036 108.25) (width 0.2) (layer "B.Cu") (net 15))
 (arc (start 144.683792 90.823971) (mid 143.504213 92.589336) (end 143.09 94.671727) (width 0.2) (layer "B.Cu") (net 15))
 (arc (start 152.190833 106.656207) (mid 153.956198 107.835786) (end 156.038589 108.25) (width 0.2) (layer "B.Cu") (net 15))
 (arc (start 146.28 104.65) (mid 145.272971 104.449689) (end 144.419253 103.879253) (width 0.2) (layer "B.Cu") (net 15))
 (arc (start 165.745535 104.497986) (mid 165.66716 104.892) (end 165.443969 105.22603) (width 0.2) (layer "B.Cu") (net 15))
 (arc (start 138.076884 103.276615) (mid 139.99532 102.895014) (end 141.621692 101.808307) (width 0.2) (layer "B.Cu") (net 15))
 (arc (start 149.047313 102.708485) (mid 148.899523 103.45147) (end 148.478656 104.081343) (width 0.2) (layer "B.Cu") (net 15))
 (arc (start 149.047313 102.708485) (mid 149.195101 103.45147) (end 149.615969 104.081343) (width 0.2) (layer "B.Cu") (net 15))
 (arc (start 143.09 101.445) (mid 143.293066 102.465886) (end 143.871352 103.331352) (width 0.2) (layer "B.Cu") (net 15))
 (arc (start 150.458658 87.347378) (mid 152.541048 86.933164) (end 154.306414 85.753585) (width 0.2) (layer "B.Cu") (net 15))
 (arc (start 148.100918 104.459081) (mid 147.889447 104.600381) (end 147.64 104.65) (width 0.2) (layer "B.Cu") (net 15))
 (segment (start 141.71 80.55) (end 141.707133 80.547133) (width 0.2) (layer "F.Cu") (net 3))
 (segment (start 141.700213 80.544267) (end 139.827539 80.544267) (width 0.2) (layer "F.Cu") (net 3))
 (via (at 141.71 80.55) (size 0.6) (drill 0.3) (layers "F.Cu" "B.Cu") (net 3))
 (arc (start 141.700213 80.544267) (mid 141.703958 80.545011) (end 141.707133 80.547133) (width 0.2) (layer "F.Cu") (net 3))
 (segment (start 144.616557 78.847378) (end 148.160386 78.847378) (width 0.2) (layer "B.Cu") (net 3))
 (segment (start 141.71 80.55) (end 142.561311 79.698689) (width 0.2) (layer "B.Cu") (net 3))
 (arc (start 144.616557 78.847378) (mid 143.504265 79.068626) (end 142.561311 79.698689) (width 0.2) (layer "B.Cu") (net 3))
 (segment (start 138.101271 83.079255) (end 139.987027 83.079255) (width 0.2) (layer "F.Cu") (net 4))
 (segment (start 138.100372 83.079627) (end 138.1 83.08) (width 0.2) (layer "F.Cu") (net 4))
 (via (at 138.1 83.08) (size 0.6) (drill 0.3) (layers "F.Cu" "B.Cu") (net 4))
 (arc (start 138.100372 83.079627) (mid 138.100784 83.079351) (end 138.101271 83.079255) (width 0.2) (layer "F.Cu") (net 4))
 (segment (start 137.015 83.995) (end 137.869895 83.140104) (width 0.2) (layer "B.Cu") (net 4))
 (segment (start 138.1 83.08) (end 138.015 83.08) (width 0.2) (layer "B.Cu") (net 4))
 (segment (start 134.623064 91.231287) (end 134.623064 94.776615) (width 0.2) (layer "B.Cu") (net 4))
 (segment (start 136.1 86.204005) (end 136.1 87.665648) (width 0.2) (layer "B.Cu") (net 4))
 (arc (start 134.623064 91.231287) (mid 134.814985 90.266432) (end 135.361532 89.448468) (width 0.2) (layer "B.Cu") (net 4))
 (arc (start 137.869895 83.140104) (mid 137.936469 83.09562) (end 138.015 83.08) (width 0.2) (layer "B.Cu") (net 4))
 (arc (start 137.015 83.995) (mid 136.3378 85.0085) (end 136.1 86.204005) (width 0.2) (layer "B.Cu") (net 4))
 (arc (start 136.1 87.665648) (mid 135.908078 88.630503) (end 135.361532 89.448468) (width 0.2) (layer "B.Cu") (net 4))
 (segment (start 145.952245 91.56) (end 146.81 91.56) (width 0.2) (layer "F.Cu") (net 6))
 (segment (start 140.994862 88.149231) (end 140.306003 88.149231) (width 0.2) (layer "F.Cu") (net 6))
 (segment (start 142.170817 88.636327) (end 144.487965 90.953475) (width 0.2) (layer "F.Cu") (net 6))
 (via (at 146.81 91.56) (size 0.6) (drill 0.3) (layers "F.Cu" "B.Cu") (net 6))
 (arc (start 145.952245 91.56) (mid 145.159782 91.402369) (end 144.487965 90.953475) (width 0.2) (layer "F.Cu") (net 6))
 (arc (start 142.170817 88.636327) (mid 141.631284 88.275823) (end 140.994862 88.149231) (width 0.2) (layer "F.Cu") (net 6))
 (segment (start 146.81 91.56) (end 147.11081 91.56) (width 0.2) (layer "B.Cu") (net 6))
 (segment (start 147.624326 91.772705) (end 149.047313 93.195692) (width 0.2) (layer "B.Cu") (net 6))
 (arc (start 147.624326 91.772705) (mid 147.388722 91.61528) (end 147.11081 91.56) (width 0.2) (layer "B.Cu") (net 6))
 (segment (start 141.690824 84.669171) (end 141.526304 84.83369) (width 0.2) (layer "F.Cu") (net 5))
 (segment (start 141.526304 84.83369) (end 141.498092 84.861902) (width 0.2) (layer "F.Cu") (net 5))
 (segment (start 143.698277 83.68) (end 143.561555 83.68) (width 0.2) (layer "F.Cu") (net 5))
 (segment (start 144.210984 83.68) (end 144.381887 83.68) (width 0.2) (layer "F.Cu") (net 5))
 (segment (start 141.281903 85.078092) (end 141.173808 85.186187) (width 0.2) (layer "F.Cu") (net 5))
 (segment (start 143.834999 83.68) (end 143.698277 83.68) (width 0.2) (layer "F.Cu") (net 5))
 (segment (start 140.446136 85.614243) (end 140.146515 85.614243) (width 0.2) (layer "F.Cu") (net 5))
 (segment (start 141.498092 84.861902) (end 141.389998 84.969997) (width 0.2) (layer "F.Cu") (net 5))
 (segment (start 154.35 91) (end 147.783068 84.433068) (width 0.2) (layer "F.Cu") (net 5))
 (segment (start 143.561555 83.68) (end 143.424833 83.68) (width 0.2) (layer "F.Cu") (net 5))
 (segment (start 141.173808 85.186187) (end 141.065713 85.294282) (width 0.2) (layer "F.Cu") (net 5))
 (segment (start 143.971721 83.68) (end 143.834999 83.68) (width 0.2) (layer "F.Cu") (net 5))
 (segment (start 141.038691 85.321305) (end 140.984644 85.375354) (width 0.2) (layer "F.Cu") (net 5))
 (segment (start 144.928776 83.68) (end 144.381887 83.68) (width 0.2) (layer "F.Cu") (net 5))
 (segment (start 141.690824 84.669171) (end 141.929282 84.430715) (width 0.2) (layer "F.Cu") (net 5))
 (segment (start 141.065713 85.294282) (end 141.038691 85.321305) (width 0.2) (layer "F.Cu") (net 5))
 (segment (start 143.288111 83.68) (end 143.322291 83.68) (width 0.2) (layer "F.Cu") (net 5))
 (segment (start 142.143094 84.216905) (end 141.929282 84.430715) (width 0.2) (layer "F.Cu") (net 5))
 (segment (start 144.005901 83.68) (end 143.971721 83.68) (width 0.2) (layer "F.Cu") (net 5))
 (segment (start 140.984644 85.375354) (end 140.957621 85.402378) (width 0.2) (layer "F.Cu") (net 5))
 (segment (start 142.25 84.11) (end 142.143094 84.216905) (width 0.2) (layer "F.Cu") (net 5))
 (segment (start 143.390652 83.68) (end 143.322291 83.68) (width 0.2) (layer "F.Cu") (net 5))
 (segment (start 141.389998 84.969997) (end 141.281903 85.078092) (width 0.2) (layer "F.Cu") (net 5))
 (segment (start 143.390652 83.68) (end 143.424833 83.68) (width 0.2) (layer "F.Cu") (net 5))
 (segment (start 144.210984 83.68) (end 144.005901 83.68) (width 0.2) (layer "F.Cu") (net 5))
 (segment (start 145.965 83.68) (end 144.928776 83.68) (width 0.2) (layer "F.Cu") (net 5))
 (via (at 154.35 91) (size 0.6) (drill 0.3) (layers "F.Cu" "B.Cu") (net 5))
 (arc (start 140.446136 85.614243) (mid 140.722949 85.559181) (end 140.957621 85.402378) (width 0.2) (layer "F.Cu") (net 5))
 (arc (start 142.25 84.11) (mid 142.726289 83.791753) (end 143.288111 83.68) (width 0.2) (layer "F.Cu") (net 5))
 (arc (start 145.965 83.68) (mid 146.948931 83.875715) (end 147.783068 84.433068) (width 0.2) (layer "F.Cu") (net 5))
 (segment (start 161.175471 95.571508) (end 165.745535 95.571508) (width 0.2) (layer "B.Cu") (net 5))
 (segment (start 157.327715 93.977715) (end 154.35 91) (width 0.2) (layer "B.Cu") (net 5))
 (arc (start 157.327715 93.977715) (mid 159.09308 95.157294) (end 161.175471 95.571508) (width 0.2) (layer "B.Cu") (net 5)))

